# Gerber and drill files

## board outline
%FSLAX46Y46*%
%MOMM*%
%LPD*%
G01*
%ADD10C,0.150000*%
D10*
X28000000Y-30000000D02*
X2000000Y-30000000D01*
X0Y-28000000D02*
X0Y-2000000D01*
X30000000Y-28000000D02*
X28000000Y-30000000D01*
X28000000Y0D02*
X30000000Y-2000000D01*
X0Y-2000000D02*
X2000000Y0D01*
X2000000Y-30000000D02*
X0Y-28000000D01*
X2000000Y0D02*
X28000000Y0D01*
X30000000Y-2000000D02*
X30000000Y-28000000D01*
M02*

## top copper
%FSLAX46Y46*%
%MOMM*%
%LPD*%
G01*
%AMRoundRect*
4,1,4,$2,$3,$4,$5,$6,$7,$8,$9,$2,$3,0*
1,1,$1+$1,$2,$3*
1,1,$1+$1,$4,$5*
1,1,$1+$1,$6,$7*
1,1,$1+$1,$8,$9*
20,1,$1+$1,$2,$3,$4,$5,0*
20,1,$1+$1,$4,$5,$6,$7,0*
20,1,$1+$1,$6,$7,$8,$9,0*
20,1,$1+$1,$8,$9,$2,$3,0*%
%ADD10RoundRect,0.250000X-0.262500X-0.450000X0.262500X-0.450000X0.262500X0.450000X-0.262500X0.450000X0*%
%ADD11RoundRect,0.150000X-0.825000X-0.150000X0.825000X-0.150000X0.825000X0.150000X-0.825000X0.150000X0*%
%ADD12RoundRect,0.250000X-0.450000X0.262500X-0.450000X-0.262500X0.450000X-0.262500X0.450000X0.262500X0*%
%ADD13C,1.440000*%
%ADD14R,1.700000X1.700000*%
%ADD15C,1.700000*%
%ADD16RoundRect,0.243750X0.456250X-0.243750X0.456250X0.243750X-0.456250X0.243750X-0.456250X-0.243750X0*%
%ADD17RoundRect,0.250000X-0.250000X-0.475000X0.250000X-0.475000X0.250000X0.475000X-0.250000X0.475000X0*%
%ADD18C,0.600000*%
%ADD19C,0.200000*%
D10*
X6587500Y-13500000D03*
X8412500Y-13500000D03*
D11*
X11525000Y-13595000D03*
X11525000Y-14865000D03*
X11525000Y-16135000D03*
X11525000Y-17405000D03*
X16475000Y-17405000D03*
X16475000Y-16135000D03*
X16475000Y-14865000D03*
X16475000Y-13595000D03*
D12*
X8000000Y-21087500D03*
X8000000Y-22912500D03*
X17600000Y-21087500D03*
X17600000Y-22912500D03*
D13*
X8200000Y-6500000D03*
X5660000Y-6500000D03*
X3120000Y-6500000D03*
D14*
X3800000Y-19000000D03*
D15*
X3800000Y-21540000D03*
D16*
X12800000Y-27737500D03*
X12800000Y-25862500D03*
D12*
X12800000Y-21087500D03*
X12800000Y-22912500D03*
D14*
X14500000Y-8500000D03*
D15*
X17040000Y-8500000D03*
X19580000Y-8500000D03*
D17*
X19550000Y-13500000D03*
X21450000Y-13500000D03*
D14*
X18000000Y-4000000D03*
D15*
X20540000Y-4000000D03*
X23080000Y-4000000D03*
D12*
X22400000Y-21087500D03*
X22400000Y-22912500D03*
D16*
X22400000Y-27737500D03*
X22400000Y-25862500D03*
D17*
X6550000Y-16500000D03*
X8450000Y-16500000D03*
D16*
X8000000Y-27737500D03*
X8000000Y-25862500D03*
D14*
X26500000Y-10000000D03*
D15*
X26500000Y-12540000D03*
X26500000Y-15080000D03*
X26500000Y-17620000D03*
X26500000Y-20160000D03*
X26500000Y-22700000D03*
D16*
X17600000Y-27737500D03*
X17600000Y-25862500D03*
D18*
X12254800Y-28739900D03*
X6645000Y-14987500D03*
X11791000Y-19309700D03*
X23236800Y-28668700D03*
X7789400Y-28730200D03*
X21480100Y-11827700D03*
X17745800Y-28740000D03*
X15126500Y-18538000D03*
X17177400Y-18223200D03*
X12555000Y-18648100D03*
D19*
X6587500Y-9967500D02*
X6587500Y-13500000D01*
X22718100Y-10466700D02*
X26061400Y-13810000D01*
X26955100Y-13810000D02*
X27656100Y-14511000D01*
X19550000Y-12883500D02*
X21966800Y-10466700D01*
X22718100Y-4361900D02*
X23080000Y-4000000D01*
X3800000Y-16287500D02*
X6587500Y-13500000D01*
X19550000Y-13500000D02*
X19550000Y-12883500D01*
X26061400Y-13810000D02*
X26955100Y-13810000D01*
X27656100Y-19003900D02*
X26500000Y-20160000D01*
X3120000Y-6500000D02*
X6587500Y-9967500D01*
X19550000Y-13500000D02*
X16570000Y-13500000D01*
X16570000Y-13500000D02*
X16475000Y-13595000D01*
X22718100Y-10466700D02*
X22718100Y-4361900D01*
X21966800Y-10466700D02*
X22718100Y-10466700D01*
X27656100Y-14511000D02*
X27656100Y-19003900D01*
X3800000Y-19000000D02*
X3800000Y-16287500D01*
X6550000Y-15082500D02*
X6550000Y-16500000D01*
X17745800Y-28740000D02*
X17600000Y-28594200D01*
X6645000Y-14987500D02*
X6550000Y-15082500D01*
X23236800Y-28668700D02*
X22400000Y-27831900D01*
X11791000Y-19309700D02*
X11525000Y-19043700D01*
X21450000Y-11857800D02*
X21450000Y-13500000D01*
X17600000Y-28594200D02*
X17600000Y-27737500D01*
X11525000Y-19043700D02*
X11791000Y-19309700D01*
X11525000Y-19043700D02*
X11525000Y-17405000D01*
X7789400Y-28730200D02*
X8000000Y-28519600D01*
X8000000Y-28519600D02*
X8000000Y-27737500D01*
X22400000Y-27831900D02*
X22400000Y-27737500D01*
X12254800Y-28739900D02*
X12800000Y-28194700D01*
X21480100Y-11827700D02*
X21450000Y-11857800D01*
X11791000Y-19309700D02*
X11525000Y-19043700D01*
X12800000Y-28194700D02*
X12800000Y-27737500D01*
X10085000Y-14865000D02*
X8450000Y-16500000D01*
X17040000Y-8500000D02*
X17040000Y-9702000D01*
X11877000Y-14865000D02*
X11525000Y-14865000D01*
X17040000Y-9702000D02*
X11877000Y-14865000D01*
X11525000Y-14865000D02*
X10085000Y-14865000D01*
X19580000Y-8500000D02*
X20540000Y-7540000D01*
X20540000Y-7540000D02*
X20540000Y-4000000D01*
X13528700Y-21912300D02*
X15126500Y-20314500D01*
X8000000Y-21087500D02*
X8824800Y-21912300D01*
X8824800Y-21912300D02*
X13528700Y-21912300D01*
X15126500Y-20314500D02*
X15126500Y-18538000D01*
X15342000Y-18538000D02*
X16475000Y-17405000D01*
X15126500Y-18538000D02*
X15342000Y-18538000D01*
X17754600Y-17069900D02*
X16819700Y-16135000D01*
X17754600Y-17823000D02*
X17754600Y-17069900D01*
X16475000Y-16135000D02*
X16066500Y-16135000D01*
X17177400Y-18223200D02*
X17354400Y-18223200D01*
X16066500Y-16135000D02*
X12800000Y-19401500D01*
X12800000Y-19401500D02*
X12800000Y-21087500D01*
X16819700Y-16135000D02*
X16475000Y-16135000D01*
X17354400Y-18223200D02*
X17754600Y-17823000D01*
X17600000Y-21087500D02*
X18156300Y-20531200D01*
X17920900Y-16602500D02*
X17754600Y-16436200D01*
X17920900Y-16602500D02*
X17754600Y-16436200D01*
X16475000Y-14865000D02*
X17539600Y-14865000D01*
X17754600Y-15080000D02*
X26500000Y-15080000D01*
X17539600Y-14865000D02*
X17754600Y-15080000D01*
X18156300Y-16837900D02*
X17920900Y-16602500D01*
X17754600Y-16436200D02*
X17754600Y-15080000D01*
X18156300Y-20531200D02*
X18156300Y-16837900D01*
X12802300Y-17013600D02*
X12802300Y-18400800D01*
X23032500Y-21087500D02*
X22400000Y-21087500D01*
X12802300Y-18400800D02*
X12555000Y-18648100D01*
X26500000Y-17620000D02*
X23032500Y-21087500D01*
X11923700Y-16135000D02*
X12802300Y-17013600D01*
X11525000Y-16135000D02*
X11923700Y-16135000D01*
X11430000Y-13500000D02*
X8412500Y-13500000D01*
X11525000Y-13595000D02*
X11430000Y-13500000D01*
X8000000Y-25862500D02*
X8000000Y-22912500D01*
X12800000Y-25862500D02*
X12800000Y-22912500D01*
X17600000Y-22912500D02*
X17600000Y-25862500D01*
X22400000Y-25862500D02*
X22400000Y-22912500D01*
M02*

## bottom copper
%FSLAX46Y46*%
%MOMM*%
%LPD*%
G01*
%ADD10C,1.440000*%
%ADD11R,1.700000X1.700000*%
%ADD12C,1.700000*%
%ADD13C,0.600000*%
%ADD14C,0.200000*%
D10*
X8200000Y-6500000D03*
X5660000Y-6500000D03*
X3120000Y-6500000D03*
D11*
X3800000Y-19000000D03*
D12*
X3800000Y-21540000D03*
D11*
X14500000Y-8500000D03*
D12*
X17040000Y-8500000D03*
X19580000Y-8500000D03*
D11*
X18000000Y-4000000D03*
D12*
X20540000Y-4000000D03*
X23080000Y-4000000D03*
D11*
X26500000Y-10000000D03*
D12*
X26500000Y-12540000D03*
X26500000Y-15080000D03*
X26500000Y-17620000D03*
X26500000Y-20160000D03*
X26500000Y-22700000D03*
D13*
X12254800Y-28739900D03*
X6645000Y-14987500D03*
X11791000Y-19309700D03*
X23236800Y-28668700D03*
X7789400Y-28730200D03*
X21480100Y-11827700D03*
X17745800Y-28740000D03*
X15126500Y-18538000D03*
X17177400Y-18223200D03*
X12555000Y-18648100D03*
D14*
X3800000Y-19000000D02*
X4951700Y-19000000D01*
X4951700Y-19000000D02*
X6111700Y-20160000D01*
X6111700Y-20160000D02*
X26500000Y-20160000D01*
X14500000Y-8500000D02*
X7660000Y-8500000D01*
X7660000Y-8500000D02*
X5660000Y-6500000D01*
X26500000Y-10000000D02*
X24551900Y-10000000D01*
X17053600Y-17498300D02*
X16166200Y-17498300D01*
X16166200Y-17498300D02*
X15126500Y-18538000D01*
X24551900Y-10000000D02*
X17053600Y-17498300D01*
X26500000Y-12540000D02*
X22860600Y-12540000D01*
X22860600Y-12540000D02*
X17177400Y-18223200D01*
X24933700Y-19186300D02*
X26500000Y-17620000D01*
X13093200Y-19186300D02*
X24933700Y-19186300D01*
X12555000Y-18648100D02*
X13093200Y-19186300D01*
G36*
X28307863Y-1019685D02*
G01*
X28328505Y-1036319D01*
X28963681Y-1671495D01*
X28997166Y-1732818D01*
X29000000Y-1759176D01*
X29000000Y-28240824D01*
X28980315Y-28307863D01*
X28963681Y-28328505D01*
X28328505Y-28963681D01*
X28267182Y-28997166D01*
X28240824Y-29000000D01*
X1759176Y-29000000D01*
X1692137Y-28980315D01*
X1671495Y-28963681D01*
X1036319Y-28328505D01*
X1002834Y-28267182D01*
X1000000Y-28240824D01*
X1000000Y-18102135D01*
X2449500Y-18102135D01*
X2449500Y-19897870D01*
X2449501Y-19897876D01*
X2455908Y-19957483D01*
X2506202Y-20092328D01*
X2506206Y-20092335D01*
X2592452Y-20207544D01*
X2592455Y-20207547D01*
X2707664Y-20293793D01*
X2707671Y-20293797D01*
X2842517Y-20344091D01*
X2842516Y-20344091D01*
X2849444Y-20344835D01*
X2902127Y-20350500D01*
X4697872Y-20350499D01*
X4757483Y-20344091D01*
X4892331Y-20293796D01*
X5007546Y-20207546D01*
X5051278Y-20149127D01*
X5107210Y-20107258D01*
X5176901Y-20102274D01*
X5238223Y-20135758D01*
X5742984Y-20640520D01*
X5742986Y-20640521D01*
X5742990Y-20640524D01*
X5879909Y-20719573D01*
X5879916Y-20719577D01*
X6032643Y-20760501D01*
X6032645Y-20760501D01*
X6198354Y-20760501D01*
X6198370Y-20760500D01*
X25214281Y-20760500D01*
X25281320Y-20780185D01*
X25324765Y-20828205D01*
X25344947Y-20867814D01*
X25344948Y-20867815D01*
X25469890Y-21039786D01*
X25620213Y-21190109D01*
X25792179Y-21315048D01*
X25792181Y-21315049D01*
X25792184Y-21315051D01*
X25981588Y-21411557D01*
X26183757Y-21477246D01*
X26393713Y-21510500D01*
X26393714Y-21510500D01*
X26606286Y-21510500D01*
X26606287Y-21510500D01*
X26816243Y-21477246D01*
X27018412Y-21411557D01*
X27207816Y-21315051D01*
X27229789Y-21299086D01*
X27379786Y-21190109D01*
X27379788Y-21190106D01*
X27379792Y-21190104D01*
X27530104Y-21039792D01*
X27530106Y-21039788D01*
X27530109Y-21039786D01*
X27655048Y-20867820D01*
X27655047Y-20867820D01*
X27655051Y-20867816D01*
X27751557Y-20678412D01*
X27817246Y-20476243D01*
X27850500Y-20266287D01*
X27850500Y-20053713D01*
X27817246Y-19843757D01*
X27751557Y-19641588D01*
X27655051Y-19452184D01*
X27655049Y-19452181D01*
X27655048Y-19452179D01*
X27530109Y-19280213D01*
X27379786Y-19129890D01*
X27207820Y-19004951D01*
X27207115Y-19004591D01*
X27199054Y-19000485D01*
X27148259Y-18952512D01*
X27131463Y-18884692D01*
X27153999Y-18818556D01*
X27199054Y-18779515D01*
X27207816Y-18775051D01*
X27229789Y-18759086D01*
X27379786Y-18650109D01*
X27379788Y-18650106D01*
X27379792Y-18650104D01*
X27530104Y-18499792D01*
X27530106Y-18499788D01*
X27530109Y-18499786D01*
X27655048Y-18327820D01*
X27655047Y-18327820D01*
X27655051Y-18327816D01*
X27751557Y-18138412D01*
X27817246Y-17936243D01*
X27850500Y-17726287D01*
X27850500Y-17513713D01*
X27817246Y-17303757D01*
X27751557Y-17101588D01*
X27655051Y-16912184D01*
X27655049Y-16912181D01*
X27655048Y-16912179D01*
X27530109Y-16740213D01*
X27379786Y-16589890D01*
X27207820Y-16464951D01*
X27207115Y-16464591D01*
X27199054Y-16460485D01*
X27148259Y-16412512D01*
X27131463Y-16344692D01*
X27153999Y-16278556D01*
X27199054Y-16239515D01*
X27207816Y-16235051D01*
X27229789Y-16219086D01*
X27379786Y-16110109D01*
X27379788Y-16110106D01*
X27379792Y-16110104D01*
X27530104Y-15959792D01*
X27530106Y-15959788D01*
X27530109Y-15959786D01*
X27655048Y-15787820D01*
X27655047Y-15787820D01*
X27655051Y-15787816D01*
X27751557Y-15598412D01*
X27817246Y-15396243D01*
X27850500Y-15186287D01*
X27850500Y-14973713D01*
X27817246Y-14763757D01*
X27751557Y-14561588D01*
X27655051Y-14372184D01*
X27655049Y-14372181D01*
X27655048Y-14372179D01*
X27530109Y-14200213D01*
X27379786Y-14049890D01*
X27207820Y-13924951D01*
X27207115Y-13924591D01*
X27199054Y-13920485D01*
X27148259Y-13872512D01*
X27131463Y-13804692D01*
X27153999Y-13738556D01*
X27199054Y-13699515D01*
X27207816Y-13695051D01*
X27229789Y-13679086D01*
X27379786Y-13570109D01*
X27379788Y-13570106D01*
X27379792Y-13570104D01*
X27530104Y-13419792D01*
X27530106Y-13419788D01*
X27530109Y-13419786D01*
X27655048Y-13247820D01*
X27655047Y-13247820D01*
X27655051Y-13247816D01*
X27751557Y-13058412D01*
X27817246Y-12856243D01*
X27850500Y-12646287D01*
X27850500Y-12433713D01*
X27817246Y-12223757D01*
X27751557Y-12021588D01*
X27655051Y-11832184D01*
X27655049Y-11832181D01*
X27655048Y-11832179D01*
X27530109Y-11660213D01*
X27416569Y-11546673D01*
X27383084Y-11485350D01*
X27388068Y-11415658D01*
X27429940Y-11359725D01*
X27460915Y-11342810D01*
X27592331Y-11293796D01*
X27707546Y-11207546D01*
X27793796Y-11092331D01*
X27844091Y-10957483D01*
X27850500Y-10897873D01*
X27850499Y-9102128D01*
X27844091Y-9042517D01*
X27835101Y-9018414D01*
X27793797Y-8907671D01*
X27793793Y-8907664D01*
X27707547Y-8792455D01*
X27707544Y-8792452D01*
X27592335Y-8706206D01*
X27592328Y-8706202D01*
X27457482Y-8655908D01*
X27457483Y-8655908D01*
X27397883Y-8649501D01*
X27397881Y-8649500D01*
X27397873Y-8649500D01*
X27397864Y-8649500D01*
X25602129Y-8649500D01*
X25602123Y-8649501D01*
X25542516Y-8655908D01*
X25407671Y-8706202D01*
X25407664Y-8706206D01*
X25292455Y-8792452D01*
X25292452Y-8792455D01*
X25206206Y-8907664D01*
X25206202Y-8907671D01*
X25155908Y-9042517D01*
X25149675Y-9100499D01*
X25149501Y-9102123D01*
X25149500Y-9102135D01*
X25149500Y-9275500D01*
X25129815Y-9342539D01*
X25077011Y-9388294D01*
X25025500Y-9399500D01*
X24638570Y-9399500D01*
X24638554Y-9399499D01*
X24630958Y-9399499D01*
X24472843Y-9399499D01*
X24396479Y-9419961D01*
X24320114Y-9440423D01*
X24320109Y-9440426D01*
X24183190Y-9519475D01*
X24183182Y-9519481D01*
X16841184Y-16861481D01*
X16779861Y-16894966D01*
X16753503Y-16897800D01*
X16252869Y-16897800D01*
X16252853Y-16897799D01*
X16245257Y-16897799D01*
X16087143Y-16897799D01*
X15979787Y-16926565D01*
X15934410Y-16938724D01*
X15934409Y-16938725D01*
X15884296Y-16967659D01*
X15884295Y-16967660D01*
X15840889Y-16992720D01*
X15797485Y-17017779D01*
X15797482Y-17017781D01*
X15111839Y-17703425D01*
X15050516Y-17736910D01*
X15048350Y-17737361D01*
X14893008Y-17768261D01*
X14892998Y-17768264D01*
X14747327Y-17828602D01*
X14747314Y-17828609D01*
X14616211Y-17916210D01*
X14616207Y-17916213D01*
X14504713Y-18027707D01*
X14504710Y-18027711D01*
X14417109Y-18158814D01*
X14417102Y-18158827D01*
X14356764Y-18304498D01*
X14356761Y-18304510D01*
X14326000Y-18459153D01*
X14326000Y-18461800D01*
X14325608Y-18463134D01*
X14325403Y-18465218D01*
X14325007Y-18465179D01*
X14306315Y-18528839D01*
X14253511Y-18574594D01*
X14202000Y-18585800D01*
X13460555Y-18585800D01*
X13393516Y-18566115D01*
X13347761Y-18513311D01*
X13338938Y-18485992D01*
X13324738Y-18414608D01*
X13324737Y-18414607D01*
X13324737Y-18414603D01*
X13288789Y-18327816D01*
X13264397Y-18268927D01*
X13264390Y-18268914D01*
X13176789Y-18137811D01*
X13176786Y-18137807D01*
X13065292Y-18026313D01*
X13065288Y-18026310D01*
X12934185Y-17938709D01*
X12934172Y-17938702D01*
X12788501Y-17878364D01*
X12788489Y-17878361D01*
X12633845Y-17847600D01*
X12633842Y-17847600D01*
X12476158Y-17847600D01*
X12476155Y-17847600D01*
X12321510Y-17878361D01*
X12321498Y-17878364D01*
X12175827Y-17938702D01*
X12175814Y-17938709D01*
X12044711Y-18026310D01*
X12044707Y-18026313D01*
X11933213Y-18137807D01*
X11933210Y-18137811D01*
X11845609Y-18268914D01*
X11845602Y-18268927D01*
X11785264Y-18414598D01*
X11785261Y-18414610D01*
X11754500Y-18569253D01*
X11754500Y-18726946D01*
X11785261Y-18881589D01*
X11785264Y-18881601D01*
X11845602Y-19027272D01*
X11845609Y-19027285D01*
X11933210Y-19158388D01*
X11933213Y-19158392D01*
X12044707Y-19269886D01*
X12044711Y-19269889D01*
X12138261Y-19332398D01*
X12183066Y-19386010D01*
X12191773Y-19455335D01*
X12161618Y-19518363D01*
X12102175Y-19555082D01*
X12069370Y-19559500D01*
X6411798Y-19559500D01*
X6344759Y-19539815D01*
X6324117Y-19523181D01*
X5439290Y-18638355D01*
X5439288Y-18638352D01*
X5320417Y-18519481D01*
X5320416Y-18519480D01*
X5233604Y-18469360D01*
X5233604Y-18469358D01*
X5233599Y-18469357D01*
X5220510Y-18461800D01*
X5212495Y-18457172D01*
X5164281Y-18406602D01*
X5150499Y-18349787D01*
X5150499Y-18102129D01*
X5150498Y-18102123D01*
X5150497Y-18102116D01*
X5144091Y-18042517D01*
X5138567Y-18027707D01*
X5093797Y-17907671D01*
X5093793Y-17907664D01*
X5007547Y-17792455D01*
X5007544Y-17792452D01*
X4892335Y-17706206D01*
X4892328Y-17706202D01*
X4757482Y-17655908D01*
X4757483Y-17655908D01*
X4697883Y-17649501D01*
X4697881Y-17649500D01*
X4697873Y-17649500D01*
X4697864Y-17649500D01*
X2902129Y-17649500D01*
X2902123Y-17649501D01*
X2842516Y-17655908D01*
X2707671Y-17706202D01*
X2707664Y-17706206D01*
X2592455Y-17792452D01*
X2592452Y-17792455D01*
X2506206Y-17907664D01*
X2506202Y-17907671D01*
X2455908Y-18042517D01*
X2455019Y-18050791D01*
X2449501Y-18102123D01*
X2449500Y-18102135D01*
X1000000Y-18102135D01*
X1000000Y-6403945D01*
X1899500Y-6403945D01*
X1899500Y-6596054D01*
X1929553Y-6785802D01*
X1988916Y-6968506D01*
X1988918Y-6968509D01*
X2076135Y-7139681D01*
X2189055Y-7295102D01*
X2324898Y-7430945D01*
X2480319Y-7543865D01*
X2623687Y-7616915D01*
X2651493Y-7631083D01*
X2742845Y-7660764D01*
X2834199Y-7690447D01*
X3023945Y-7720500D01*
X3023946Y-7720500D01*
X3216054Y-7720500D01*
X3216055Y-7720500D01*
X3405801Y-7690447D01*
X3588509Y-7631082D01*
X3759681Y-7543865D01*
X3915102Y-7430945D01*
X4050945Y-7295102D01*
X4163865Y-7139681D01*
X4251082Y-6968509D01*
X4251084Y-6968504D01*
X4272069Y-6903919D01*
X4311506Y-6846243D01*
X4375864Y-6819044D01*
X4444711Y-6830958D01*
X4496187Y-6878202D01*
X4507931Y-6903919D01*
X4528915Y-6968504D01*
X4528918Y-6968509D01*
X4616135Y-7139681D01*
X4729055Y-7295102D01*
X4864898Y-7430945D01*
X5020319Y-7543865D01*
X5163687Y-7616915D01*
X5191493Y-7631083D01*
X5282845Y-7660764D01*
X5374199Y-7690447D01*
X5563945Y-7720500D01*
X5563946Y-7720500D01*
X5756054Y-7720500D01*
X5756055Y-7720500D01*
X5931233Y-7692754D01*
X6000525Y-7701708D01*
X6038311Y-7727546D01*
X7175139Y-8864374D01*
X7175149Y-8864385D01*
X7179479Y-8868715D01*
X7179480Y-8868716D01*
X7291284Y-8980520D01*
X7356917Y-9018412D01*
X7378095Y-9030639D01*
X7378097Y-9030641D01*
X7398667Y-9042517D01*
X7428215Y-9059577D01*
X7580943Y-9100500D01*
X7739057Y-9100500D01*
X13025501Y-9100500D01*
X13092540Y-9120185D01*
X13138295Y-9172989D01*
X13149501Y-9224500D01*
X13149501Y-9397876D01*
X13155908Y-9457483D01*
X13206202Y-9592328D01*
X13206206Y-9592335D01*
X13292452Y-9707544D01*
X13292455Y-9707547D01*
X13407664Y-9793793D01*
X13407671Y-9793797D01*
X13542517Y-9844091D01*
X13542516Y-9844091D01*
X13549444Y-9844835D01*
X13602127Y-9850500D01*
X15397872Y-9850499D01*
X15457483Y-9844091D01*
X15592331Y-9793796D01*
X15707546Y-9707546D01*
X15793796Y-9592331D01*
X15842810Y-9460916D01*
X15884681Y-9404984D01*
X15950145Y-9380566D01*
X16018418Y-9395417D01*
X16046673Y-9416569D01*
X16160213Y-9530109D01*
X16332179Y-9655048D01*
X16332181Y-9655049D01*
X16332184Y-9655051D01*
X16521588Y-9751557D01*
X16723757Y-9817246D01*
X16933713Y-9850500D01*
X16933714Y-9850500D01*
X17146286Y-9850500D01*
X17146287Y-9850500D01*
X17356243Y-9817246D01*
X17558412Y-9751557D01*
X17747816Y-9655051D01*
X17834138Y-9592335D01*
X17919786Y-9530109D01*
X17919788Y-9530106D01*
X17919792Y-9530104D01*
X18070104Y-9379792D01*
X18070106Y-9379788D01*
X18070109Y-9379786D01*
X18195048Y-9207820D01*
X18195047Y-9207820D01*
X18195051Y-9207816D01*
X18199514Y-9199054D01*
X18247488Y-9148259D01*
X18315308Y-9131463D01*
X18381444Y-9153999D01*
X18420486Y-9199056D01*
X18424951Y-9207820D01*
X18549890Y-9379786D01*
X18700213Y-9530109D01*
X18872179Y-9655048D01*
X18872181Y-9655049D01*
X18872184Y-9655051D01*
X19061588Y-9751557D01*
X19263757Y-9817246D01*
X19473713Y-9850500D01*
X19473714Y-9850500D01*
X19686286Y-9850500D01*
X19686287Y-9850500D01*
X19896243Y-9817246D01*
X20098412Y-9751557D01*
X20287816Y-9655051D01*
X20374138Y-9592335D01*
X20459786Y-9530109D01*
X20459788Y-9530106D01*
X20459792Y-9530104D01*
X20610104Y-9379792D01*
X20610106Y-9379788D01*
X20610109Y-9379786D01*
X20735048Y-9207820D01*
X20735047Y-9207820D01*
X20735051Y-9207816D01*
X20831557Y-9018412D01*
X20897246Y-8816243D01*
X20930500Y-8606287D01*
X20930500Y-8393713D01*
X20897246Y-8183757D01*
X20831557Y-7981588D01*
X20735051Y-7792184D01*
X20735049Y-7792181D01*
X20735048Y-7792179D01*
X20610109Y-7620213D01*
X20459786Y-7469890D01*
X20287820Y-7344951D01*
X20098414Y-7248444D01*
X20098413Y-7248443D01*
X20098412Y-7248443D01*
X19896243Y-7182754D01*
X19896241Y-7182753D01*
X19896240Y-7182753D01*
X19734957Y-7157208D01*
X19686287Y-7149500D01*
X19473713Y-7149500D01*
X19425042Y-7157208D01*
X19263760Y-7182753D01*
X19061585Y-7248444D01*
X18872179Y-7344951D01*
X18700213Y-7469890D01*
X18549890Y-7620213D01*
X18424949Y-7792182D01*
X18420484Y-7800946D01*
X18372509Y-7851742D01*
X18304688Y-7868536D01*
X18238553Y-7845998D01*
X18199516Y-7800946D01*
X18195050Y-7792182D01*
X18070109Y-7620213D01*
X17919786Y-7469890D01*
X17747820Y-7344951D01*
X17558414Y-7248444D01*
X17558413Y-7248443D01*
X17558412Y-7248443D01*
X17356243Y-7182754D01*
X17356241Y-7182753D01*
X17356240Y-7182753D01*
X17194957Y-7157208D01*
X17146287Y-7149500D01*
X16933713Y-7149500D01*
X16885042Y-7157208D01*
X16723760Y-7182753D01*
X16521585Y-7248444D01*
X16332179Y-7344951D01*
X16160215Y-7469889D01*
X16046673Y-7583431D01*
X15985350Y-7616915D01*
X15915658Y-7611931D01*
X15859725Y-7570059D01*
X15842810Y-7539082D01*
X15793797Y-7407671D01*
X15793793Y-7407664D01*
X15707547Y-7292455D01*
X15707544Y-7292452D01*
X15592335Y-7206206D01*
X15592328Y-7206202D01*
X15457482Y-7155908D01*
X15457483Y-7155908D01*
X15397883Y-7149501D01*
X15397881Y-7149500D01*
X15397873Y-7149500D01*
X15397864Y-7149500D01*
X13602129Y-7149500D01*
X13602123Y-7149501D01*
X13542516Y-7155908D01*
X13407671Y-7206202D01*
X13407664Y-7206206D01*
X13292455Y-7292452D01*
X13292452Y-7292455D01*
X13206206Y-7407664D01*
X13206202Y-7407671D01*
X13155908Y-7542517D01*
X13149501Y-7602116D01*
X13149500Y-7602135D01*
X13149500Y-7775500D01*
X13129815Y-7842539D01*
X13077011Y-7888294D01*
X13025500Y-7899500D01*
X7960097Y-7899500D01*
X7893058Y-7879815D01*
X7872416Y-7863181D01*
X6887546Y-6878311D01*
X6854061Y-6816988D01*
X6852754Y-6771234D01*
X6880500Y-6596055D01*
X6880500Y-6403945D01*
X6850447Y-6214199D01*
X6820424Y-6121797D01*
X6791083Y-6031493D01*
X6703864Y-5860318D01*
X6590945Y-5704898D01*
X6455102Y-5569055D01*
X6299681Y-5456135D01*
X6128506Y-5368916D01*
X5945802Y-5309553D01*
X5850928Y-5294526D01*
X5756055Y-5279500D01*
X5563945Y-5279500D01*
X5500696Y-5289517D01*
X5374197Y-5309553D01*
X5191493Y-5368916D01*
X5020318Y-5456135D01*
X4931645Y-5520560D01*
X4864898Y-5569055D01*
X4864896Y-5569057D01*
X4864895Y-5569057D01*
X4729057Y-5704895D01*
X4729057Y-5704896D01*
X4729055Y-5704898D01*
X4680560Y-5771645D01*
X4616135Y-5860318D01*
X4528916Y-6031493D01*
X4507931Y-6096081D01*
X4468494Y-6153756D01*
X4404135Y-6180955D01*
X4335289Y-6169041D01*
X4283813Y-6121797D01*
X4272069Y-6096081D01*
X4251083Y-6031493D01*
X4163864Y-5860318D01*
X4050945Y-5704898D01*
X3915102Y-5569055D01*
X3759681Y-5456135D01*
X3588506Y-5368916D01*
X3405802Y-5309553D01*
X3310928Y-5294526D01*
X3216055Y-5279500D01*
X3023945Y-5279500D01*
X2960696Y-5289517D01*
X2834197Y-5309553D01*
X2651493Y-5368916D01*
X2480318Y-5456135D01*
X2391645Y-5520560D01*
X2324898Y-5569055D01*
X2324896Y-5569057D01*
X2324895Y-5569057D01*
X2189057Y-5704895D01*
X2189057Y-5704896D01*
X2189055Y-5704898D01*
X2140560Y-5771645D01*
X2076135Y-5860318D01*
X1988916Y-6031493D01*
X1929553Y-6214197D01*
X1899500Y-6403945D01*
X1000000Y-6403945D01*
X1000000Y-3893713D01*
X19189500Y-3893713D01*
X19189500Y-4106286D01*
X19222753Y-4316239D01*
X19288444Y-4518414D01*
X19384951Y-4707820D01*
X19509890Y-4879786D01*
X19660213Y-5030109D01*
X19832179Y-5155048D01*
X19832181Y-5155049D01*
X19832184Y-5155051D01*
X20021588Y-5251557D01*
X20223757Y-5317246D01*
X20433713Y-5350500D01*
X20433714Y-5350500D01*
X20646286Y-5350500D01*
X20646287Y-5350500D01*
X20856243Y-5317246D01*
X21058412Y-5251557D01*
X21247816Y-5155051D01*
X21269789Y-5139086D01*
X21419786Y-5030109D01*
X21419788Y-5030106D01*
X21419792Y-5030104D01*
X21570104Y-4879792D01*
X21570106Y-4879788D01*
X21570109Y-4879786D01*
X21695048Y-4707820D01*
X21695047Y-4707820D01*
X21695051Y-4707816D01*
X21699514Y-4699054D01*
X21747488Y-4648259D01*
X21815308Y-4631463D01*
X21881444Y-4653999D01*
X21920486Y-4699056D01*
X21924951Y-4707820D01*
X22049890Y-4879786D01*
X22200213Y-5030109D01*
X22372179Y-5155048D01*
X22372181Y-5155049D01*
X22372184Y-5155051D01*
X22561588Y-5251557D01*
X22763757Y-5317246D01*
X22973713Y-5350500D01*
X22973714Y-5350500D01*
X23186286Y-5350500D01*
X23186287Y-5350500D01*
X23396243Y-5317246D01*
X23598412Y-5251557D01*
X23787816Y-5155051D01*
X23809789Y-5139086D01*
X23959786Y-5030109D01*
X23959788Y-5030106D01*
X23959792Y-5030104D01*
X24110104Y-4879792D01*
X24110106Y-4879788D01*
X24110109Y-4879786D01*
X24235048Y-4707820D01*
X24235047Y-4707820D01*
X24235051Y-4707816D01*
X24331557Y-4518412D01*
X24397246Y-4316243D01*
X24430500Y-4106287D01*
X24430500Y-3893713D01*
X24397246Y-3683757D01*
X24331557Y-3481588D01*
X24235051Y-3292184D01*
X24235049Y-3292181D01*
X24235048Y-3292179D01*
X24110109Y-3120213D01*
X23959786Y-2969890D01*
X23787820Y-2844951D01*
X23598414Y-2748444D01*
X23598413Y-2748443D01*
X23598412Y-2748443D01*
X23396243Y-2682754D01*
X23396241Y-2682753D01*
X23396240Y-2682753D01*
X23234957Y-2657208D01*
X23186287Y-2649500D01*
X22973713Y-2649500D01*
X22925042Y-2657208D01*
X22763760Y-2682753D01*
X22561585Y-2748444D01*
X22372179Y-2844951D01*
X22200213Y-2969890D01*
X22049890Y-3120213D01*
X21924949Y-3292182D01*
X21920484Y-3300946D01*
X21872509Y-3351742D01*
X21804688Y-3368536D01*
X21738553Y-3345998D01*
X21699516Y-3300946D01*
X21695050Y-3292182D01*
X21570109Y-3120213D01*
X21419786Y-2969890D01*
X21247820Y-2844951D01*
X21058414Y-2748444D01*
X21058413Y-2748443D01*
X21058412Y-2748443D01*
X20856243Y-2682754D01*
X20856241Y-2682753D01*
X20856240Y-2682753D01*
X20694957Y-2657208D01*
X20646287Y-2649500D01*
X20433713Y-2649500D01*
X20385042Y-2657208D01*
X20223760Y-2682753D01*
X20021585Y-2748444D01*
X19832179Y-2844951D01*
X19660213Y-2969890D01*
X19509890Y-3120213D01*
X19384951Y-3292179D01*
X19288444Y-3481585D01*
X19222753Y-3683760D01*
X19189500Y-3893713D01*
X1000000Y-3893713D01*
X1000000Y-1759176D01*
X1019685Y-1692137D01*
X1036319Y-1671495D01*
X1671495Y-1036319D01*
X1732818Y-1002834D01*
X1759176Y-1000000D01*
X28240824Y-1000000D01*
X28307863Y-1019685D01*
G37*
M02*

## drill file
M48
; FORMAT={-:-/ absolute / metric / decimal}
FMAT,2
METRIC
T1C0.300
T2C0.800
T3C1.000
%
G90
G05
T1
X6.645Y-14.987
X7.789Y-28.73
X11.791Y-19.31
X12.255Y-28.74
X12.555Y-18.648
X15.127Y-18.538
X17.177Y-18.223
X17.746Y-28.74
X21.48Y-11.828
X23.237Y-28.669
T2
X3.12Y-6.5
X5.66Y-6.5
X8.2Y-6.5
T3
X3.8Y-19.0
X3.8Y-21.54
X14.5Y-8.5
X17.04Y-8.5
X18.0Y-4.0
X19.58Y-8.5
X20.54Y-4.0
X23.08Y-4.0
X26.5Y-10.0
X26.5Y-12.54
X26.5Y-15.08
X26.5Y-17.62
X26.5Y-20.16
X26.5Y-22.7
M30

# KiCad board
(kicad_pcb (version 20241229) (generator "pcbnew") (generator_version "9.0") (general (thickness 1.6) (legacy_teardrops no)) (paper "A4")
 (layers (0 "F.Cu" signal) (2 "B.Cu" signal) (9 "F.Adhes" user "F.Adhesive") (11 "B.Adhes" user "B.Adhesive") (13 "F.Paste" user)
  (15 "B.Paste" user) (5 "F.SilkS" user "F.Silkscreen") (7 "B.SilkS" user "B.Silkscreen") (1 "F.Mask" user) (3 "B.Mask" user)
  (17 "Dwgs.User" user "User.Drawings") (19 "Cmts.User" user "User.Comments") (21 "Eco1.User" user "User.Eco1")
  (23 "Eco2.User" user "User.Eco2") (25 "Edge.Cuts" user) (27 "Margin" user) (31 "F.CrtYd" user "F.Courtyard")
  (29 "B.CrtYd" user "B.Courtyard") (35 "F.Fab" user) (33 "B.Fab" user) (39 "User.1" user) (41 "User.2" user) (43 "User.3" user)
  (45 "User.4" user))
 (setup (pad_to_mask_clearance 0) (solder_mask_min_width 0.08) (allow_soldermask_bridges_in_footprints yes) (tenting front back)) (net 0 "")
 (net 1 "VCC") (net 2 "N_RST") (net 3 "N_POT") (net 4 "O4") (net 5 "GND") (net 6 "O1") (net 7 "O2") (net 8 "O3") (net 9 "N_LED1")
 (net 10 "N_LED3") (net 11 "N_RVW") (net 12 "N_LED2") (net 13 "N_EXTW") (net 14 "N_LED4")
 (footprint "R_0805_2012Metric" (layer "F.Cu") (at 7.5 13.5)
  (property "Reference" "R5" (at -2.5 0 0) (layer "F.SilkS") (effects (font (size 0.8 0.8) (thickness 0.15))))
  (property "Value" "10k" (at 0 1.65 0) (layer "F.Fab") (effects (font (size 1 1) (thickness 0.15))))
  (pad "1" smd roundrect (at -0.9125 0) (size 1.025 1.4) (layers "F.Cu" "F.Mask" "F.Paste") (roundrect_rratio 0.243902) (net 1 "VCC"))
  (pad "2" smd roundrect (at 0.9125 0) (size 1.025 1.4) (layers "F.Cu" "F.Mask" "F.Paste") (roundrect_rratio 0.243902) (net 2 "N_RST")))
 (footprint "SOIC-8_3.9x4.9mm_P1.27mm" (layer "F.Cu") (at 14 15.5)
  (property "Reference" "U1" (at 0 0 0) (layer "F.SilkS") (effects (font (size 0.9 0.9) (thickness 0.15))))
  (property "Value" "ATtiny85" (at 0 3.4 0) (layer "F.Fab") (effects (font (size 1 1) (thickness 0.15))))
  (pad "1" smd roundrect (at -2.475 -1.905) (size 1.95 0.6) (layers "F.Cu" "F.Mask" "F.Paste") (roundrect_rratio 0.25) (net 2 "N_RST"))
  (pad "2" smd roundrect (at -2.475 -0.635) (size 1.95 0.6) (layers "F.Cu" "F.Mask" "F.Paste") (roundrect_rratio 0.25) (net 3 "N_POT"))
  (pad "3" smd roundrect (at -2.475 0.635) (size 1.95 0.6) (layers "F.Cu" "F.Mask" "F.Paste") (roundrect_rratio 0.25) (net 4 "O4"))
  (pad "4" smd roundrect (at -2.475 1.905) (size 1.95 0.6) (layers "F.Cu" "F.Mask" "F.Paste") (roundrect_rratio 0.25) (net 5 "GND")
   (zone_connect 2))
  (pad "5" smd roundrect (at 2.475 1.905) (size 1.95 0.6) (layers "F.Cu" "F.Mask" "F.Paste") (roundrect_rratio 0.25) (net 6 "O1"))
  (pad "6" smd roundrect (at 2.475 0.635) (size 1.95 0.6) (layers "F.Cu" "F.Mask" "F.Paste") (roundrect_rratio 0.25) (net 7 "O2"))
  (pad "7" smd roundrect (at 2.475 -0.635) (size 1.95 0.6) (layers "F.Cu" "F.Mask" "F.Paste") (roundrect_rratio 0.25) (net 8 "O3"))
  (pad "8" smd roundrect (at 2.475 -1.905) (size 1.95 0.6) (layers "F.Cu" "F.Mask" "F.Paste") (roundrect_rratio 0.25) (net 1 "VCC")))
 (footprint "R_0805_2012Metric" (layer "F.Cu") (at 8 22 -90)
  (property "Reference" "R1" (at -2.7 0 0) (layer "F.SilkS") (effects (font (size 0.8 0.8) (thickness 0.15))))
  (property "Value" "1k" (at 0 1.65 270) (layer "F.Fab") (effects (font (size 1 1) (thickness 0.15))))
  (pad "1" smd roundrect (at -0.9125 0 270) (size 1.025 1.4) (layers "F.Cu" "F.Mask" "F.Paste") (roundrect_rratio 0.243902) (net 6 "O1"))
  (pad "2" smd roundrect (at 0.9125 0 270) (size 1.025 1.4) (layers "F.Cu" "F.Mask" "F.Paste") (roundrect_rratio 0.243902) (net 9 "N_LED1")))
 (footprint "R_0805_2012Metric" (layer "F.Cu") (at 17.6 22 -90)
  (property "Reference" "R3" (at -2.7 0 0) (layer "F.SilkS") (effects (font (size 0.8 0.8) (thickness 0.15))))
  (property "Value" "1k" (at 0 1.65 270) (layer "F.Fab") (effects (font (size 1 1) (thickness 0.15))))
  (pad "1" smd roundrect (at -0.9125 0 270) (size 1.025 1.4) (layers "F.Cu" "F.Mask" "F.Paste") (roundrect_rratio 0.243902) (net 8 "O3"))
  (pad "2" smd roundrect (at 0.9125 0 270) (size 1.025 1.4) (layers "F.Cu" "F.Mask" "F.Paste") (roundrect_rratio 0.243902) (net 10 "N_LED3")))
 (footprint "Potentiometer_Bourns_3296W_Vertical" (layer "F.Cu") (at 8.2 6.5)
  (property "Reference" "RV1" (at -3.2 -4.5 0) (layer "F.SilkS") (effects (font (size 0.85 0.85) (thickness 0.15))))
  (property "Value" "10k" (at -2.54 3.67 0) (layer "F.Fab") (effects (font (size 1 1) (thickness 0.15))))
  (pad "1" thru_hole circle (at 0 0) (size 1.44 1.44) (drill 0.8) (layers "*.Cu" "*.Mask") (remove_unused_layers no) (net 5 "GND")
   (zone_connect 2))
  (pad "2" thru_hole circle (at -2.54 0) (size 1.44 1.44) (drill 0.8) (layers "*.Cu" "*.Mask") (remove_unused_layers no) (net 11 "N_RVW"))
  (pad "3" thru_hole circle (at -5.08 0) (size 1.44 1.44) (drill 0.8) (layers "*.Cu" "*.Mask") (remove_unused_layers no) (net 1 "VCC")))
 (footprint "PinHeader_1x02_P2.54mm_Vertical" (layer "F.Cu") (at 3.8 19)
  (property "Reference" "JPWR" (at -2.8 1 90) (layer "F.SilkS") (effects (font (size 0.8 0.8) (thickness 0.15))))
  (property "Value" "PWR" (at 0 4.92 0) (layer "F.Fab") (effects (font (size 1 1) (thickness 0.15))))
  (pad "1" thru_hole rect (at 0 0) (size 1.7 1.7) (drill 1) (layers "*.Cu" "*.Mask") (remove_unused_layers no) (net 1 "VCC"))
  (pad "2" thru_hole circle (at 0 2.54) (size 1.7 1.7) (drill 1) (layers "*.Cu" "*.Mask") (remove_unused_layers no) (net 5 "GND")
   (zone_connect 2)))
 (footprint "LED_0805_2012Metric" (layer "F.Cu") (at 12.8 26.8 90)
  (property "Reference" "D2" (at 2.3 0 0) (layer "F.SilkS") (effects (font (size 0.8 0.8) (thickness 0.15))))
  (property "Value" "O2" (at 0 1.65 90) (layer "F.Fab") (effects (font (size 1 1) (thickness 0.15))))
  (pad "1" smd roundrect (at -0.9375 0 90) (size 0.975 1.4) (layers "F.Cu" "F.Mask" "F.Paste") (roundrect_rratio 0.25) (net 5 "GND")
   (zone_connect 2))
  (pad "2" smd roundrect (at 0.9375 0 90) (size 0.975 1.4) (layers "F.Cu" "F.Mask" "F.Paste") (roundrect_rratio 0.25) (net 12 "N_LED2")))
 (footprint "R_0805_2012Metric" (layer "F.Cu") (at 12.8 22 -90)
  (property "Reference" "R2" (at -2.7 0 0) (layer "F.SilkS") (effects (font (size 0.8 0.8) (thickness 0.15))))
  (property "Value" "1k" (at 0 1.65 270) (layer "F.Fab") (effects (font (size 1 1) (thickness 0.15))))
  (pad "1" smd roundrect (at -0.9125 0 270) (size 1.025 1.4) (layers "F.Cu" "F.Mask" "F.Paste") (roundrect_rratio 0.243902) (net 7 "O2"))
  (pad "2" smd roundrect (at 0.9125 0 270) (size 1.025 1.4) (layers "F.Cu" "F.Mask" "F.Paste") (roundrect_rratio 0.243902) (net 12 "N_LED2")))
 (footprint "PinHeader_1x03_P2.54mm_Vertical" (layer "F.Cu") (at 14.5 8.5 90)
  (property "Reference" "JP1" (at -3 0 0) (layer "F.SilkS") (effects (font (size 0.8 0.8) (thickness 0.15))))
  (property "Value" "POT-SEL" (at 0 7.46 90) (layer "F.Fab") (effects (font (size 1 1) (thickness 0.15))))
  (pad "1" thru_hole rect (at 0 0 90) (size 1.7 1.7) (drill 1) (layers "*.Cu" "*.Mask") (remove_unused_layers no) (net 11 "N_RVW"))
  (pad "2" thru_hole circle (at 0 2.54 90) (size 1.7 1.7) (drill 1) (layers "*.Cu" "*.Mask") (remove_unused_layers no) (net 3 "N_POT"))
  (pad "3" thru_hole circle (at 0 5.08 90) (size 1.7 1.7) (drill 1) (layers "*.Cu" "*.Mask") (remove_unused_layers no) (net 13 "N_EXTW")))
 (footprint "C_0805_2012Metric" (layer "F.Cu") (at 20.5 13.5)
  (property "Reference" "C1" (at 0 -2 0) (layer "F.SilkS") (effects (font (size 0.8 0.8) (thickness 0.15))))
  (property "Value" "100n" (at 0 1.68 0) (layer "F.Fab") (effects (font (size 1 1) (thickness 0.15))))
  (pad "1" smd roundrect (at -0.95 0) (size 1 1.45) (layers "F.Cu" "F.Mask" "F.Paste") (roundrect_rratio 0.25) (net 1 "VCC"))
  (pad "2" smd roundrect (at 0.95 0) (size 1 1.45) (layers "F.Cu" "F.Mask" "F.Paste") (roundrect_rratio 0.25) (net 5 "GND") (zone_connect 2)))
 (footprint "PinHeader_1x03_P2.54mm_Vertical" (layer "F.Cu") (at 18 4 90)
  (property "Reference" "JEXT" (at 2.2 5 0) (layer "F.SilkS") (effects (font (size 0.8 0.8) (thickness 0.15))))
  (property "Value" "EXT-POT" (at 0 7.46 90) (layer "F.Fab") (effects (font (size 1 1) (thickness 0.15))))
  (pad "1" thru_hole rect (at 0 0 90) (size 1.7 1.7) (drill 1) (layers "*.Cu" "*.Mask") (remove_unused_layers no) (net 5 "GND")
   (zone_connect 2))
  (pad "2" thru_hole circle (at 0 2.54 90) (size 1.7 1.7) (drill 1) (layers "*.Cu" "*.Mask") (remove_unused_layers no) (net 13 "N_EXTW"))
  (pad "3" thru_hole circle (at 0 5.08 90) (size 1.7 1.7) (drill 1) (layers "*.Cu" "*.Mask") (remove_unused_layers no) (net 1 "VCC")))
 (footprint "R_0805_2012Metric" (layer "F.Cu") (at 22.4 22 -90)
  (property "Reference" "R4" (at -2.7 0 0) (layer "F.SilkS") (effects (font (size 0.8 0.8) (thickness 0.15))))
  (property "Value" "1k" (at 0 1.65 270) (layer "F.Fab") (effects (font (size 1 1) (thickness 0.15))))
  (pad "1" smd roundrect (at -0.9125 0 270) (size 1.025 1.4) (layers "F.Cu" "F.Mask" "F.Paste") (roundrect_rratio 0.243902) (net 4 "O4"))
  (pad "2" smd roundrect (at 0.9125 0 270) (size 1.025 1.4) (layers "F.Cu" "F.Mask" "F.Paste") (roundrect_rratio 0.243902) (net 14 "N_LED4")))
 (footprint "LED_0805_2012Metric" (layer "F.Cu") (at 22.4 26.8 90)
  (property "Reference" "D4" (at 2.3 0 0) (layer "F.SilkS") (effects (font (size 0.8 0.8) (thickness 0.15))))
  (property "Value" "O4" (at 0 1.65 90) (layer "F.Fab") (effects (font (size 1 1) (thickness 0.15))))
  (pad "1" smd roundrect (at -0.9375 0 90) (size 0.975 1.4) (layers "F.Cu" "F.Mask" "F.Paste") (roundrect_rratio 0.25) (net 5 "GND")
   (zone_connect 2))
  (pad "2" smd roundrect (at 0.9375 0 90) (size 0.975 1.4) (layers "F.Cu" "F.Mask" "F.Paste") (roundrect_rratio 0.25) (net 14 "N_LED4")))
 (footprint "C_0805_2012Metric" (layer "F.Cu") (at 7.5 16.5)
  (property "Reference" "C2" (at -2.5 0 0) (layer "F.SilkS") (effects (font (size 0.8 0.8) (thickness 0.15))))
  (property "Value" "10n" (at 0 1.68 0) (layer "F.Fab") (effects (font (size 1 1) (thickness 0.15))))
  (pad "1" smd roundrect (at -0.95 0) (size 1 1.45) (layers "F.Cu" "F.Mask" "F.Paste") (roundrect_rratio 0.25) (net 5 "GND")
   (zone_connect 2))
  (pad "2" smd roundrect (at 0.95 0) (size 1 1.45) (layers "F.Cu" "F.Mask" "F.Paste") (roundrect_rratio 0.25) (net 3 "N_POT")))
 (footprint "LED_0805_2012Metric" (layer "F.Cu") (at 8 26.8 90)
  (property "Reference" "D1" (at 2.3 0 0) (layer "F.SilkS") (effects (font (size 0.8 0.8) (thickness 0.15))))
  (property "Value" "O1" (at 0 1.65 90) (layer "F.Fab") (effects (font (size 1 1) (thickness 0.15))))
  (pad "1" smd roundrect (at -0.9375 0 90) (size 0.975 1.4) (layers "F.Cu" "F.Mask" "F.Paste") (roundrect_rratio 0.25) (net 5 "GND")
   (zone_connect 2))
  (pad "2" smd roundrect (at 0.9375 0 90) (size 0.975 1.4) (layers "F.Cu" "F.Mask" "F.Paste") (roundrect_rratio 0.25) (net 9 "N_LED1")))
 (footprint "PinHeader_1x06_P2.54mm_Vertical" (layer "F.Cu") (at 26.5 10)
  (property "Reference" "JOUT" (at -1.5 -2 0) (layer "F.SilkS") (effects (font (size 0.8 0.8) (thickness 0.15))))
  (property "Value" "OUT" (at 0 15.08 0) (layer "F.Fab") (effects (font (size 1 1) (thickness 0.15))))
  (pad "1" thru_hole rect (at 0 0) (size 1.7 1.7) (drill 1) (layers "*.Cu" "*.Mask") (remove_unused_layers no) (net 6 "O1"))
  (pad "2" thru_hole circle (at 0 2.54) (size 1.7 1.7) (drill 1) (layers "*.Cu" "*.Mask") (remove_unused_layers no) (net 7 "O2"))
  (pad "3" thru_hole circle (at 0 5.08) (size 1.7 1.7) (drill 1) (layers "*.Cu" "*.Mask") (remove_unused_layers no) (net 8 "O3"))
  (pad "4" thru_hole circle (at 0 7.62) (size 1.7 1.7) (drill 1) (layers "*.Cu" "*.Mask") (remove_unused_layers no) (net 4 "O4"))
  (pad "5" thru_hole circle (at 0 10.16) (size 1.7 1.7) (drill 1) (layers "*.Cu" "*.Mask") (remove_unused_layers no) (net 1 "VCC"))
  (pad "6" thru_hole circle (at 0 12.7) (size 1.7 1.7) (drill 1) (layers "*.Cu" "*.Mask") (remove_unused_layers no) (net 5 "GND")
   (zone_connect 2)))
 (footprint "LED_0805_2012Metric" (layer "F.Cu") (at 17.6 26.8 90)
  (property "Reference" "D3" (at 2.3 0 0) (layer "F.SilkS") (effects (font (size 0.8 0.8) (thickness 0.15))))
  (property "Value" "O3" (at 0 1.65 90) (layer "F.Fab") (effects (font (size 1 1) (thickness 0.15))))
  (pad "1" smd roundrect (at -0.9375 0 90) (size 0.975 1.4) (layers "F.Cu" "F.Mask" "F.Paste") (roundrect_rratio 0.25) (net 5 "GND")
   (zone_connect 2))
  (pad "2" smd roundrect (at 0.9375 0 90) (size 0.975 1.4) (layers "F.Cu" "F.Mask" "F.Paste") (roundrect_rratio 0.25) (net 10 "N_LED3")))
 (gr_line (start 28 30) (end 2 30) (stroke (width 0.15) (type default)) (layer "Edge.Cuts"))
 (gr_line (start 0 28) (end 0 2) (stroke (width 0.15) (type default)) (layer "Edge.Cuts"))
 (gr_line (start 30 28) (end 28 30) (stroke (width 0.15) (type default)) (layer "Edge.Cuts"))
 (gr_line (start 28 0) (end 30 2) (stroke (width 0.15) (type default)) (layer "Edge.Cuts"))
 (gr_line (start 0 2) (end 2 0) (stroke (width 0.15) (type default)) (layer "Edge.Cuts"))
 (gr_line (start 2 30) (end 0 28) (stroke (width 0.15) (type default)) (layer "Edge.Cuts"))
 (gr_line (start 2 0) (end 28 0) (stroke (width 0.15) (type default)) (layer "Edge.Cuts"))
 (gr_line (start 30 2) (end 30 28) (stroke (width 0.15) (type default)) (layer "Edge.Cuts"))
 (segment (start 6.5875 9.9675) (end 6.5875 13.5) (width 0.2) (layer "F.Cu") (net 1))
 (segment (start 22.7181 10.4667) (end 26.0614 13.81) (width 0.2) (layer "F.Cu") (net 1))
 (segment (start 26.9551 13.81) (end 27.6561 14.511) (width 0.2) (layer "F.Cu") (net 1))
 (segment (start 19.55 12.8835) (end 21.9668 10.4667) (width 0.2) (layer "F.Cu") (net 1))
 (segment (start 22.7181 4.3619) (end 23.08 4) (width 0.2) (layer "F.Cu") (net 1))
 (segment (start 3.8 16.2875) (end 6.5875 13.5) (width 0.2) (layer "F.Cu") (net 1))
 (segment (start 19.55 13.5) (end 19.55 12.8835) (width 0.2) (layer "F.Cu") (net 1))
 (segment (start 26.0614 13.81) (end 26.9551 13.81) (width 0.2) (layer "F.Cu") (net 1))
 (segment (start 27.6561 19.0039) (end 26.5 20.16) (width 0.2) (layer "F.Cu") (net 1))
 (segment (start 3.12 6.5) (end 6.5875 9.9675) (width 0.2) (layer "F.Cu") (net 1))
 (segment (start 19.55 13.5) (end 16.57 13.5) (width 0.2) (layer "F.Cu") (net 1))
 (segment (start 16.57 13.5) (end 16.475 13.595) (width 0.2) (layer "F.Cu") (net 1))
 (segment (start 22.7181 10.4667) (end 22.7181 4.3619) (width 0.2) (layer "F.Cu") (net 1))
 (segment (start 21.9668 10.4667) (end 22.7181 10.4667) (width 0.2) (layer "F.Cu") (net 1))
 (segment (start 27.6561 14.511) (end 27.6561 19.0039) (width 0.2) (layer "F.Cu") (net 1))
 (segment (start 3.8 19) (end 3.8 16.2875) (width 0.2) (layer "F.Cu") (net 1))
 (segment (start 3.8 19) (end 4.9517 19) (width 0.2) (layer "B.Cu") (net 1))
 (segment (start 4.9517 19) (end 6.1117 20.16) (width 0.2) (layer "B.Cu") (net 1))
 (segment (start 6.1117 20.16) (end 26.5 20.16) (width 0.2) (layer "B.Cu") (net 1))
 (segment (start 6.55 15.0825) (end 6.55 16.5) (width 0.2) (layer "F.Cu") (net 5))
 (segment (start 17.7458 28.74) (end 17.6 28.5942) (width 0.2) (layer "F.Cu") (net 5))
 (segment (start 6.645 14.9875) (end 6.55 15.0825) (width 0.2) (layer "F.Cu") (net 5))
 (segment (start 23.2368 28.6687) (end 22.4 27.8319) (width 0.2) (layer "F.Cu") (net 5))
 (segment (start 11.791 19.3097) (end 11.525 19.0437) (width 0.2) (layer "F.Cu") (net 5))
 (segment (start 21.45 11.8578) (end 21.45 13.5) (width 0.2) (layer "F.Cu") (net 5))
 (segment (start 17.6 28.5942) (end 17.6 27.7375) (width 0.2) (layer "F.Cu") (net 5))
 (segment (start 11.525 19.0437) (end 11.791 19.3097) (width 0.2) (layer "F.Cu") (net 5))
 (segment (start 11.525 19.0437) (end 11.525 17.405) (width 0.2) (layer "F.Cu") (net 5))
 (segment (start 7.7894 28.7302) (end 8 28.5196) (width 0.2) (layer "F.Cu") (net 5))
 (segment (start 8 28.5196) (end 8 27.7375) (width 0.2) (layer "F.Cu") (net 5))
 (segment (start 22.4 27.8319) (end 22.4 27.7375) (width 0.2) (layer "F.Cu") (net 5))
 (segment (start 12.2548 28.7399) (end 12.8 28.1947) (width 0.2) (layer "F.Cu") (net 5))
 (segment (start 21.4801 11.8277) (end 21.45 11.8578) (width 0.2) (layer "F.Cu") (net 5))
 (segment (start 11.791 19.3097) (end 11.525 19.0437) (width 0.2) (layer "F.Cu") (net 5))
 (segment (start 12.8 28.1947) (end 12.8 27.7375) (width 0.2) (layer "F.Cu") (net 5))
 (via (at 12.2548 28.7399) (size 0.6) (drill 0.3) (layers "F.Cu" "B.Cu") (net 5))
 (via (at 6.645 14.9875) (size 0.6) (drill 0.3) (layers "F.Cu" "B.Cu") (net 5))
 (via (at 11.791 19.3097) (size 0.6) (drill 0.3) (layers "F.Cu" "B.Cu") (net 5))
 (via (at 23.2368 28.6687) (size 0.6) (drill 0.3) (layers "F.Cu" "B.Cu") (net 5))
 (via (at 7.7894 28.7302) (size 0.6) (drill 0.3) (layers "F.Cu" "B.Cu") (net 5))
 (via (at 21.4801 11.8277) (size 0.6) (drill 0.3) (layers "F.Cu" "B.Cu") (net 5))
 (via (at 17.7458 28.74) (size 0.6) (drill 0.3) (layers "F.Cu" "B.Cu") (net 5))
 (segment (start 10.085 14.865) (end 8.45 16.5) (width 0.2) (layer "F.Cu") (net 3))
 (segment (start 17.04 8.5) (end 17.04 9.702) (width 0.2) (layer "F.Cu") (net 3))
 (segment (start 11.877 14.865) (end 11.525 14.865) (width 0.2) (layer "F.Cu") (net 3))
 (segment (start 17.04 9.702) (end 11.877 14.865) (width 0.2) (layer "F.Cu") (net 3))
 (segment (start 11.525 14.865) (end 10.085 14.865) (width 0.2) (layer "F.Cu") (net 3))
 (segment (start 14.5 8.5) (end 7.66 8.5) (width 0.2) (layer "B.Cu") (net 11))
 (segment (start 7.66 8.5) (end 5.66 6.5) (width 0.2) (layer "B.Cu") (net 11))
 (segment (start 19.58 8.5) (end 20.54 7.54) (width 0.2) (layer "F.Cu") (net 13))
 (segment (start 20.54 7.54) (end 20.54 4) (width 0.2) (layer "F.Cu") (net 13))
 (segment (start 13.5287 21.9123) (end 15.1265 20.3145) (width 0.2) (layer "F.Cu") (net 6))
 (segment (start 8 21.0875) (end 8.8248 21.9123) (width 0.2) (layer "F.Cu") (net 6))
 (segment (start 8.8248 21.9123) (end 13.5287 21.9123) (width 0.2) (layer "F.Cu") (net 6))
 (segment (start 15.1265 20.3145) (end 15.1265 18.538) (width 0.2) (layer "F.Cu") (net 6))
 (segment (start 15.342 18.538) (end 16.475 17.405) (width 0.2) (layer "F.Cu") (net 6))
 (segment (start 15.1265 18.538) (end 15.342 18.538) (width 0.2) (layer "F.Cu") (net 6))
 (via (at 15.1265 18.538) (size 0.6) (drill 0.3) (layers "F.Cu" "B.Cu") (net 6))
 (segment (start 26.5 10) (end 24.5519 10) (width 0.2) (layer "B.Cu") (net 6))
 (segment (start 17.0536 17.4983) (end 16.1662 17.4983) (width 0.2) (layer "B.Cu") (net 6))
 (segment (start 16.1662 17.4983) (end 15.1265 18.538) (width 0.2) (layer "B.Cu") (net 6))
 (segment (start 24.5519 10) (end 17.0536 17.4983) (width 0.2) (layer "B.Cu") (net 6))
 (segment (start 17.7546 17.0699) (end 16.8197 16.135) (width 0.2) (layer "F.Cu") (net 7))
 (segment (start 17.7546 17.823) (end 17.7546 17.0699) (width 0.2) (layer "F.Cu") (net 7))
 (segment (start 16.475 16.135) (end 16.0665 16.135) (width 0.2) (layer "F.Cu") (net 7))
 (segment (start 17.1774 18.2232) (end 17.3544 18.2232) (width 0.2) (layer "F.Cu") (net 7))
 (segment (start 16.0665 16.135) (end 12.8 19.4015) (width 0.2) (layer "F.Cu") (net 7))
 (segment (start 12.8 19.4015) (end 12.8 21.0875) (width 0.2) (layer "F.Cu") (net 7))
 (segment (start 16.8197 16.135) (end 16.475 16.135) (width 0.2) (layer "F.Cu") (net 7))
 (segment (start 17.3544 18.2232) (end 17.7546 17.823) (width 0.2) (layer "F.Cu") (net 7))
 (via (at 17.1774 18.2232) (size 0.6) (drill 0.3) (layers "F.Cu" "B.Cu") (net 7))
 (segment (start 26.5 12.54) (end 22.8606 12.54) (width 0.2) (layer "B.Cu") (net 7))
 (segment (start 22.8606 12.54) (end 17.1774 18.2232) (width 0.2) (layer "B.Cu") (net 7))
 (segment (start 17.6 21.0875) (end 18.1563 20.5312) (width 0.2) (layer "F.Cu") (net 8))
 (segment (start 17.9209 16.6025) (end 17.7546 16.4362) (width 0.2) (layer "F.Cu") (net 8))
 (segment (start 17.9209 16.6025) (end 17.7546 16.4362) (width 0.2) (layer "F.Cu") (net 8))
 (segment (start 16.475 14.865) (end 17.5396 14.865) (width 0.2) (layer "F.Cu") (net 8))
 (segment (start 17.7546 15.08) (end 26.5 15.08) (width 0.2) (layer "F.Cu") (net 8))
 (segment (start 17.5396 14.865) (end 17.7546 15.08) (width 0.2) (layer "F.Cu") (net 8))
 (segment (start 18.1563 16.8379) (end 17.9209 16.6025) (width 0.2) (layer "F.Cu") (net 8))
 (segment (start 17.7546 16.4362) (end 17.7546 15.08) (width 0.2) (layer "F.Cu") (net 8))
 (segment (start 18.1563 20.5312) (end 18.1563 16.8379) (width 0.2) (layer "F.Cu") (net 8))
 (segment (start 12.8023 17.0136) (end 12.8023 18.4008) (width 0.2) (layer "F.Cu") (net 4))
 (segment (start 23.0325 21.0875) (end 22.4 21.0875) (width 0.2) (layer "F.Cu") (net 4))
 (segment (start 12.8023 18.4008) (end 12.555 18.6481) (width 0.2) (layer "F.Cu") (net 4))
 (segment (start 26.5 17.62) (end 23.0325 21.0875) (width 0.2) (layer "F.Cu") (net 4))
 (segment (start 11.9237 16.135) (end 12.8023 17.0136) (width 0.2) (layer "F.Cu") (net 4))
 (segment (start 11.525 16.135) (end 11.9237 16.135) (width 0.2) (layer "F.Cu") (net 4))
 (via (at 12.555 18.6481) (size 0.6) (drill 0.3) (layers "F.Cu" "B.Cu") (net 4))
 (segment (start 24.9337 19.1863) (end 26.5 17.62) (width 0.2) (layer "B.Cu") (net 4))
 (segment (start 13.0932 19.1863) (end 24.9337 19.1863) (width 0.2) (layer "B.Cu") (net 4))
 (segment (start 12.555 18.6481) (end 13.0932 19.1863) (width 0.2) (layer "B.Cu") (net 4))
 (segment (start 11.43 13.5) (end 8.4125 13.5) (width 0.2) (layer "F.Cu") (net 2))
 (segment (start 11.525 13.595) (end 11.43 13.5) (width 0.2) (layer "F.Cu") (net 2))
 (segment (start 8 25.8625) (end 8 22.9125) (width 0.2) (layer "F.Cu") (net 9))
 (segment (start 12.8 25.8625) (end 12.8 22.9125) (width 0.2) (layer "F.Cu") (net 12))
 (segment (start 17.6 22.9125) (end 17.6 25.8625) (width 0.2) (layer "F.Cu") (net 10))
 (segment (start 22.4 25.8625) (end 22.4 22.9125) (width 0.2) (layer "F.Cu") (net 14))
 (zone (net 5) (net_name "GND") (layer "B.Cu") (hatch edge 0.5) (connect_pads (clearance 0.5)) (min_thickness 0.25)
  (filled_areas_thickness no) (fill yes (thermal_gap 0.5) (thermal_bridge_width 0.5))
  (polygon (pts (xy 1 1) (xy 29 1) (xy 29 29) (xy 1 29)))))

